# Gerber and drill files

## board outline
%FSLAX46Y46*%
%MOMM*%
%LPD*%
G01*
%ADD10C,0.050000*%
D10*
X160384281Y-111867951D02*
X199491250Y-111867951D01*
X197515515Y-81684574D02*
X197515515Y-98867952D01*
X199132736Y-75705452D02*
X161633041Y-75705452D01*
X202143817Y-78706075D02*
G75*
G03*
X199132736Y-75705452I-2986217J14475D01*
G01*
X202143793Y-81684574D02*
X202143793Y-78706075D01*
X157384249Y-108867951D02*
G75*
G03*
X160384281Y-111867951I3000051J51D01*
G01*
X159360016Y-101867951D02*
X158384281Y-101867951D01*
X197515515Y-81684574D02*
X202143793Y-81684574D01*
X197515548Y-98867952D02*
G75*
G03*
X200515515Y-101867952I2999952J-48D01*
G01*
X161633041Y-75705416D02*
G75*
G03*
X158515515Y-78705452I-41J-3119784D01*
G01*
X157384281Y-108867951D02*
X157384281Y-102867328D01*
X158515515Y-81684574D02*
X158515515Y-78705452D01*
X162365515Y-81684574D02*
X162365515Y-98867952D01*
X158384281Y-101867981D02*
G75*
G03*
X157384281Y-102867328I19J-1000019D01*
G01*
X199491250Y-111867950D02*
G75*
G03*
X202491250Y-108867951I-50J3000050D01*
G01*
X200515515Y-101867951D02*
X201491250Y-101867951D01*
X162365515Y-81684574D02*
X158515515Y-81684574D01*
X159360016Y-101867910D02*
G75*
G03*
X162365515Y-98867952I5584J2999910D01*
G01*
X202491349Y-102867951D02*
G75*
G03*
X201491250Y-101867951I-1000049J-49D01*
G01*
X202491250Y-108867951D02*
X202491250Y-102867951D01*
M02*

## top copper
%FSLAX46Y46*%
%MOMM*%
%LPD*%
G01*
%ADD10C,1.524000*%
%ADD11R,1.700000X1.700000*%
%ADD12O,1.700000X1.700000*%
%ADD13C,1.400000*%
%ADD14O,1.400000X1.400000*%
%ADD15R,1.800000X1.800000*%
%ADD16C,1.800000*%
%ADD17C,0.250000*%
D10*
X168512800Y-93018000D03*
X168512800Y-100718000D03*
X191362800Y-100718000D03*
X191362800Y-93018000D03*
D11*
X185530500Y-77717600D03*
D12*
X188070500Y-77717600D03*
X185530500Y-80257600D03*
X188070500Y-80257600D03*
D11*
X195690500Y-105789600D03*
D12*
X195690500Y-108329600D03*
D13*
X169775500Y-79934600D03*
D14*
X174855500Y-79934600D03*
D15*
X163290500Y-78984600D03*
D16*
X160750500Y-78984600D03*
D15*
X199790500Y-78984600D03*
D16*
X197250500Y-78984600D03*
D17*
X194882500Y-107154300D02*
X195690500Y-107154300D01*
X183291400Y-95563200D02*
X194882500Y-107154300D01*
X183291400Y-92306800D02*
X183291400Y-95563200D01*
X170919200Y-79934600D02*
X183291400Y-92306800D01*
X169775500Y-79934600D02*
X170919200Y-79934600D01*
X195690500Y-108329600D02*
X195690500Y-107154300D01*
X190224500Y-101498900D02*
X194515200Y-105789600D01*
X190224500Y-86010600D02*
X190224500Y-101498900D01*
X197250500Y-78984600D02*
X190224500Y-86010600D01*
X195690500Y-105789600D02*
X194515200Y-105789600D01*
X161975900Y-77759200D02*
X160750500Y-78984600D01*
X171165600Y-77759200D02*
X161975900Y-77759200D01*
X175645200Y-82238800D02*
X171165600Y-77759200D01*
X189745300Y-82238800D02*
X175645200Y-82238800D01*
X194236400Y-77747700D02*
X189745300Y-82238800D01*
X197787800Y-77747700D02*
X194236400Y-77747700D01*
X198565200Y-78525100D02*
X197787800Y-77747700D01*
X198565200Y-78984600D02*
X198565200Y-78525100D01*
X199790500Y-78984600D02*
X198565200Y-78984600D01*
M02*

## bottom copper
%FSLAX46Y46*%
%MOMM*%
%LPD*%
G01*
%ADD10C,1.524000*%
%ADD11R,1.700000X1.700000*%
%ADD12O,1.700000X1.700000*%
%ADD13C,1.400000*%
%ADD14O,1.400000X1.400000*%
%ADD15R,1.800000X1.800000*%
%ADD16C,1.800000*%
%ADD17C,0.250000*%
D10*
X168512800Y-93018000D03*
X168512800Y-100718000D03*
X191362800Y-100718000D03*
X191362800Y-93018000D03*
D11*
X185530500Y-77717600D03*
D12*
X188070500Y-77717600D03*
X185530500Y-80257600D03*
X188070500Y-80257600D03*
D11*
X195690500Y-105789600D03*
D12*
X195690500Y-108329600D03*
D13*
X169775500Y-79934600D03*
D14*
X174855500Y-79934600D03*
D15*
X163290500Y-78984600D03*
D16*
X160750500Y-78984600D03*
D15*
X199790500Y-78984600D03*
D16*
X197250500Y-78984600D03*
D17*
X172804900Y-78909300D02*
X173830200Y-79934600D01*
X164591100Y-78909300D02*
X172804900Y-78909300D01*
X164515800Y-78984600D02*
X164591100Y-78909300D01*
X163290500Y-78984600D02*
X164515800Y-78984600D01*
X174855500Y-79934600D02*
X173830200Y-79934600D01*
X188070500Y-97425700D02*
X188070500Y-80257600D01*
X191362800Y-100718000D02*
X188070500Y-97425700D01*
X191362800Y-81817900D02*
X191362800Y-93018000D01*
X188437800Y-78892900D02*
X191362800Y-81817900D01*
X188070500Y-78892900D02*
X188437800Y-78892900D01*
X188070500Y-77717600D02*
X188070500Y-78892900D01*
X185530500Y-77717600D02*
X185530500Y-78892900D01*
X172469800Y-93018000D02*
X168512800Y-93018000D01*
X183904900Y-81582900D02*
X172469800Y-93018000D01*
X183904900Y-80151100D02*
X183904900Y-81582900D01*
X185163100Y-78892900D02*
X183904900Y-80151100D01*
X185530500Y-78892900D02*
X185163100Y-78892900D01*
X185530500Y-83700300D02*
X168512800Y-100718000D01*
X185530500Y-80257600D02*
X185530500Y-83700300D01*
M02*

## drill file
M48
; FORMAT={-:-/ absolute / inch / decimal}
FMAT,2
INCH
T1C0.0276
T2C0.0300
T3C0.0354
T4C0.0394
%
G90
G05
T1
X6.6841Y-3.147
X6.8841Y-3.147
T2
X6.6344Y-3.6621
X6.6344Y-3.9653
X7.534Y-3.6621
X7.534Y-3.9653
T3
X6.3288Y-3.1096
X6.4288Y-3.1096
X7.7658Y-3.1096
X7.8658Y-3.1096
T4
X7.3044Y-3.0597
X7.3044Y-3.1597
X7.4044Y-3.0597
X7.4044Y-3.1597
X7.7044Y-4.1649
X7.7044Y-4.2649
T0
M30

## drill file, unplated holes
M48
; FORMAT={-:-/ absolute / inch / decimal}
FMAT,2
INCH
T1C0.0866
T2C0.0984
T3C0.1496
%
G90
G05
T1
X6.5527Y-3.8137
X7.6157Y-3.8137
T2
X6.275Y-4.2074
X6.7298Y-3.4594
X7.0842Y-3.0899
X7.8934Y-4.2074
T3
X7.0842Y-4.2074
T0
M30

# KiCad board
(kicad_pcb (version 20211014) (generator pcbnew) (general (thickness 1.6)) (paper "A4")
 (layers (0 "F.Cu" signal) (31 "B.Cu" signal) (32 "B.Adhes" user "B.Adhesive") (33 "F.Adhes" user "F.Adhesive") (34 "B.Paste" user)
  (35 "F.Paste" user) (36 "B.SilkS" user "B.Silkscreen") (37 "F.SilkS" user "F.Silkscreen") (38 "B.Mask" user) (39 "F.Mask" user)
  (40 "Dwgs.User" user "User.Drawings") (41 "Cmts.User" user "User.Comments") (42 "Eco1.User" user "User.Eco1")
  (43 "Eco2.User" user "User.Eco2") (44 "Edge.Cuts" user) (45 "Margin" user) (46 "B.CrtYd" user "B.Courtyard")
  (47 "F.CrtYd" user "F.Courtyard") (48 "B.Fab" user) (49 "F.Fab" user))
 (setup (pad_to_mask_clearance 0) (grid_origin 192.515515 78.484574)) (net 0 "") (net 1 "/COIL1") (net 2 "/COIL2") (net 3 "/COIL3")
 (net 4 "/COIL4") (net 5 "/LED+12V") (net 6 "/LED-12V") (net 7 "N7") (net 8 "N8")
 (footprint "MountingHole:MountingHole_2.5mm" (layer "F.Cu") (at 179.9378 78.4846)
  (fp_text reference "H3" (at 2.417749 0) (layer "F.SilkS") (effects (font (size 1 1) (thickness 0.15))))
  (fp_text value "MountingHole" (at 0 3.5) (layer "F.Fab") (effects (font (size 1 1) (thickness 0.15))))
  (pad "" np_thru_hole circle locked (at 0 0) (size 2.5 2.5) (drill 2.5) (layers *.Cu *.Mask)))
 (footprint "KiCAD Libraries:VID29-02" (layer "F.Cu") (at 180.1028 96.868)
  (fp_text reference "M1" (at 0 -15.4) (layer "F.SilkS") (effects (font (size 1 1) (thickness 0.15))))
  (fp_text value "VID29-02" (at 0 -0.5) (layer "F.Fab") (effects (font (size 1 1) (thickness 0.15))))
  (pad "" np_thru_hole circle locked (at -9.165 -9) (size 2.5 2.5) (drill 2.5) (layers *.Cu *.Mask))
  (pad "" np_thru_hole circle locked (at 13.335 0) (size 2.2 2.2) (drill 2.2) (layers *.Cu *.Mask))
  (pad "" np_thru_hole circle locked (at -0.165 10) (size 3.8 3.8) (drill 3.8) (layers *.Cu *.Mask))
  (pad "" np_thru_hole circle locked (at -13.665 0) (size 2.2 2.2) (drill 2.2) (layers *.Cu *.Mask))
  (pad "1" thru_hole circle locked (at -11.59 -3.85) (size 1.524 1.524) (drill 0.762) (layers *.Cu *.Mask) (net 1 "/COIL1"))
  (pad "2" thru_hole circle locked (at -11.59 3.85) (size 1.524 1.524) (drill 0.762) (layers *.Cu *.Mask) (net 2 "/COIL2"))
  (pad "3" thru_hole circle locked (at 11.26 3.85) (size 1.524 1.524) (drill 0.762) (layers *.Cu *.Mask) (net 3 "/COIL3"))
  (pad "4" thru_hole circle locked (at 11.26 -3.85) (size 1.524 1.524) (drill 0.762) (layers *.Cu *.Mask) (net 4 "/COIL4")))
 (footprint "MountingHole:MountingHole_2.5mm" (layer "F.Cu") (at 159.3843 106.868)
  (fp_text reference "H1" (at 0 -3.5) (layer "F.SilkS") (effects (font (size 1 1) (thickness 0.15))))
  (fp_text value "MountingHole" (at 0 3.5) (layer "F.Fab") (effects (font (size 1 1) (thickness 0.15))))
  (pad "" np_thru_hole circle locked (at 0 0) (size 2.5 2.5) (drill 2.5) (layers *.Cu *.Mask)))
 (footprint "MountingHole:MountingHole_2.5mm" (layer "F.Cu") (at 200.4913 106.868)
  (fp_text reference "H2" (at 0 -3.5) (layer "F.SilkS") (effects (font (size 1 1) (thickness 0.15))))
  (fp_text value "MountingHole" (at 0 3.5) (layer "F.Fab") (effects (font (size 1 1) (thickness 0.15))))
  (pad "" np_thru_hole circle locked (at 0 0) (size 2.5 2.5) (drill 2.5) (layers *.Cu *.Mask)))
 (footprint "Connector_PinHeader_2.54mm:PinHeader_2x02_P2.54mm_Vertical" (layer "F.Cu") (at 185.5305 77.7176)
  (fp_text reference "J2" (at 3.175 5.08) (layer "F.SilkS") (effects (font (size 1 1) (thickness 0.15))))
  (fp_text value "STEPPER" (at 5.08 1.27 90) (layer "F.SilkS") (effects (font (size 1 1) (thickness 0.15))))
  (pad "1" thru_hole rect locked (at 0 0) (size 1.7 1.7) (drill 1) (layers *.Cu *.Mask) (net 1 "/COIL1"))
  (pad "2" thru_hole oval locked (at 2.54 0) (size 1.7 1.7) (drill 1) (layers *.Cu *.Mask) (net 4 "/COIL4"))
  (pad "3" thru_hole oval locked (at 0 2.54) (size 1.7 1.7) (drill 1) (layers *.Cu *.Mask) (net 2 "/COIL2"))
  (pad "4" thru_hole oval locked (at 2.54 2.54) (size 1.7 1.7) (drill 1) (layers *.Cu *.Mask) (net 3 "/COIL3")))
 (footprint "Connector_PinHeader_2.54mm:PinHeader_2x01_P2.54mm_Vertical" (layer "F.Cu") (at 195.6905 105.7896 -90)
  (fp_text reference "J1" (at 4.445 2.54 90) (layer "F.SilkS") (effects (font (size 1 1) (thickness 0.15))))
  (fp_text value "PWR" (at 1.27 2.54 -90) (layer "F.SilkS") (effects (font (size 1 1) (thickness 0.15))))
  (pad "1" thru_hole rect locked (at 0 0 270) (size 1.7 1.7) (drill 1) (layers *.Cu *.Mask) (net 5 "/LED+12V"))
  (pad "2" thru_hole oval locked (at 2.54 0 270) (size 1.7 1.7) (drill 1) (layers *.Cu *.Mask) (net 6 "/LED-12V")))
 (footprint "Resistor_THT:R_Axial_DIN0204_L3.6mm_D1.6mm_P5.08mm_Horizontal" (layer "F.Cu") (at 169.7755 79.9346)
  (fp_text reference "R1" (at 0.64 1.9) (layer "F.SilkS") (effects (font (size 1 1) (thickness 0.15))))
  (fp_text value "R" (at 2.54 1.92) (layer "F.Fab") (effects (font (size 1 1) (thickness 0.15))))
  (pad "1" thru_hole circle (at 0 0) (size 1.4 1.4) (drill 0.7) (layers *.Cu *.Mask) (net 6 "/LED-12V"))
  (pad "2" thru_hole oval (at 5.08 0) (size 1.4 1.4) (drill 0.7) (layers *.Cu *.Mask) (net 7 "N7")))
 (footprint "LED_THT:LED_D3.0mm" (layer "B.Cu") (at 163.2905 78.9846 180)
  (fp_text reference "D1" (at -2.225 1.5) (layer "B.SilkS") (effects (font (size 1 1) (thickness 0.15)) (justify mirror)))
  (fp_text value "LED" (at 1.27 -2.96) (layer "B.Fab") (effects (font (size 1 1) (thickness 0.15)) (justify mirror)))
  (pad "1" thru_hole rect (at 0 0 180) (size 1.8 1.8) (drill 0.9) (layers *.Cu *.Mask) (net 7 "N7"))
  (pad "2" thru_hole circle (at 2.54 0 180) (size 1.8 1.8) (drill 0.9) (layers *.Cu *.Mask) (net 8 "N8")))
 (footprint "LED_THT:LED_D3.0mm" (layer "B.Cu") (at 199.7905 78.9846 180)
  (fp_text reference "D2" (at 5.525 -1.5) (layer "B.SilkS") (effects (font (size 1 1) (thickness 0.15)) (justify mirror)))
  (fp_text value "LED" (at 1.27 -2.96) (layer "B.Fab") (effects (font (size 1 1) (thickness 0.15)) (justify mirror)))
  (pad "1" thru_hole rect (at 0 0 180) (size 1.8 1.8) (drill 0.9) (layers *.Cu *.Mask) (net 8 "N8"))
  (pad "2" thru_hole circle (at 2.54 0 180) (size 1.8 1.8) (drill 0.9) (layers *.Cu *.Mask) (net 5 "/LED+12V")))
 (gr_line (start 160.384281 111.867951) (end 199.49125 111.867951) (layer "Edge.Cuts") (width 0.05))
 (gr_line (start 197.515515 81.684574) (end 197.515515 98.867952) (layer "Edge.Cuts") (width 0.05))
 (gr_line (start 199.132736 75.705452) (end 161.633041 75.705452) (layer "Edge.Cuts") (width 0.05))
 (gr_arc (start 199.132736 75.705452) (mid 201.265508 76.576339) (end 202.143793 78.706075) (layer "Edge.Cuts") (width 0.05))
 (gr_line (start 202.143793 81.684574) (end 202.143793 78.706075) (layer "Edge.Cuts") (width 0.05))
 (gr_arc (start 160.384281 111.867951) (mid 158.262961 110.989271) (end 157.384281 108.867951) (layer "Edge.Cuts") (width 0.05))
 (gr_line (start 159.360016 101.867951) (end 158.384281 101.867951) (layer "Edge.Cuts") (width 0.05))
 (gr_line (start 197.515515 81.684574) (end 202.143793 81.684574) (layer "Edge.Cuts") (width 0.05))
 (gr_arc (start 200.515515 101.867952) (mid 198.394195 100.989272) (end 197.515515 98.867952) (layer "Edge.Cuts") (width 0.05))
 (gr_arc (start 158.515515 78.705452) (mid 159.469751 76.577243) (end 161.633041 75.705452) (layer "Edge.Cuts") (width 0.05))
 (gr_line (start 157.384281 108.867951) (end 157.384281 102.867328) (layer "Edge.Cuts") (width 0.05))
 (gr_line (start 158.515515 81.684574) (end 158.515515 78.705452) (layer "Edge.Cuts") (width 0.05))
 (gr_line (start 162.365515 81.684574) (end 162.365515 98.867952) (layer "Edge.Cuts") (width 0.05))
 (gr_arc (start 157.384281 102.867328) (mid 157.677399 102.160628) (end 158.384281 101.867951) (layer "Edge.Cuts") (width 0.05))
 (gr_arc (start 202.49125 108.867951) (mid 201.61257 110.989271) (end 199.49125 111.867951) (layer "Edge.Cuts") (width 0.05))
 (gr_line (start 200.515515 101.867951) (end 201.49125 101.867951) (layer "Edge.Cuts") (width 0.05))
 (gr_line (start 162.365515 81.684574) (end 158.515515 81.684574) (layer "Edge.Cuts") (width 0.05))
 (gr_arc (start 162.365515 98.867952) (mid 161.484904 100.991231) (end 159.360016 101.867951) (layer "Edge.Cuts") (width 0.05))
 (gr_arc (start 201.49125 101.867951) (mid 202.198357 102.160844) (end 202.49125 102.867951) (layer "Edge.Cuts") (width 0.05))
 (gr_line (start 202.49125 108.867951) (end 202.49125 102.867951) (layer "Edge.Cuts") (width 0.05))
 (segment (start 185.5305 83.7003) (end 168.5128 100.718) (width 0.25) (layer "B.Cu") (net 2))
 (segment (start 185.5305 80.2576) (end 185.5305 83.7003) (width 0.25) (layer "B.Cu") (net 2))
 (segment (start 185.5305 77.7176) (end 185.5305 78.8929) (width 0.25) (layer "B.Cu") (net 1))
 (segment (start 172.4698 93.018) (end 168.5128 93.018) (width 0.25) (layer "B.Cu") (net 1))
 (segment (start 183.9049 80.1511) (end 183.9049 81.5829) (width 0.25) (layer "B.Cu") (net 1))
 (segment (start 185.1631 78.8929) (end 183.9049 80.1511) (width 0.25) (layer "B.Cu") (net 1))
 (segment (start 185.5305 78.8929) (end 185.1631 78.8929) (width 0.25) (layer "B.Cu") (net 1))
 (segment (start 183.9049 81.5829) (end 172.4698 93.018) (width 0.25) (layer "B.Cu") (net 1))
 (segment (start 191.3628 81.8179) (end 191.3628 93.018) (width 0.25) (layer "B.Cu") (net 4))
 (segment (start 188.4378 78.8929) (end 191.3628 81.8179) (width 0.25) (layer "B.Cu") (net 4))
 (segment (start 188.0705 77.7176) (end 188.0705 78.8929) (width 0.25) (layer "B.Cu") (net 4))
 (segment (start 188.0705 78.8929) (end 188.4378 78.8929) (width 0.25) (layer "B.Cu") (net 4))
 (segment (start 188.0705 97.4257) (end 188.0705 80.2576) (width 0.25) (layer "B.Cu") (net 3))
 (segment (start 191.3628 100.718) (end 188.0705 97.4257) (width 0.25) (layer "B.Cu") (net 3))
 (segment (start 198.5652 78.5251) (end 197.7878 77.7477) (width 0.25) (layer "F.Cu") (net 8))
 (segment (start 197.7878 77.7477) (end 194.2364 77.7477) (width 0.25) (layer "F.Cu") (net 8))
 (segment (start 198.5652 78.9846) (end 198.5652 78.5251) (width 0.25) (layer "F.Cu") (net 8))
 (segment (start 199.7905 78.9846) (end 198.5652 78.9846) (width 0.25) (layer "F.Cu") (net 8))
 (segment (start 194.2364 77.7477) (end 189.7453 82.2388) (width 0.25) (layer "F.Cu") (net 8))
 (segment (start 161.9759 77.7592) (end 160.7505 78.9846) (width 0.25) (layer "F.Cu") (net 8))
 (segment (start 189.7453 82.2388) (end 175.6452 82.2388) (width 0.25) (layer "F.Cu") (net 8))
 (segment (start 171.1656 77.7592) (end 161.9759 77.7592) (width 0.25) (layer "F.Cu") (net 8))
 (segment (start 175.6452 82.2388) (end 171.1656 77.7592) (width 0.25) (layer "F.Cu") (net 8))
 (segment (start 197.2505 78.9846) (end 190.2245 86.0106) (width 0.25) (layer "F.Cu") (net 5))
 (segment (start 195.6905 105.7896) (end 194.5152 105.7896) (width 0.25) (layer "F.Cu") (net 5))
 (segment (start 190.2245 86.0106) (end 190.2245 101.4989) (width 0.25) (layer "F.Cu") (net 5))
 (segment (start 190.2245 101.4989) (end 194.5152 105.7896) (width 0.25) (layer "F.Cu") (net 5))
 (segment (start 170.9192 79.9346) (end 183.2914 92.3068) (width 0.25) (layer "F.Cu") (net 6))
 (segment (start 195.6905 108.3296) (end 195.6905 107.1543) (width 0.25) (layer "F.Cu") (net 6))
 (segment (start 169.7755 79.9346) (end 170.9192 79.9346) (width 0.25) (layer "F.Cu") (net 6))
 (segment (start 183.2914 95.5632) (end 194.8825 107.1543) (width 0.25) (layer "F.Cu") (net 6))
 (segment (start 194.8825 107.1543) (end 195.6905 107.1543) (width 0.25) (layer "F.Cu") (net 6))
 (segment (start 183.2914 92.3068) (end 183.2914 95.5632) (width 0.25) (layer "F.Cu") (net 6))
 (segment (start 174.8555 79.9346) (end 173.8302 79.9346) (width 0.25) (layer "B.Cu") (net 7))
 (segment (start 164.5911 78.9093) (end 172.8049 78.9093) (width 0.25) (layer "B.Cu") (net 7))
 (segment (start 172.8049 78.9093) (end 173.8302 79.9346) (width 0.25) (layer "B.Cu") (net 7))
 (segment (start 163.2905 78.9846) (end 164.5158 78.9846) (width 0.25) (layer "B.Cu") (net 7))
 (segment (start 164.5158 78.9846) (end 164.5911 78.9093) (width 0.25) (layer "B.Cu") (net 7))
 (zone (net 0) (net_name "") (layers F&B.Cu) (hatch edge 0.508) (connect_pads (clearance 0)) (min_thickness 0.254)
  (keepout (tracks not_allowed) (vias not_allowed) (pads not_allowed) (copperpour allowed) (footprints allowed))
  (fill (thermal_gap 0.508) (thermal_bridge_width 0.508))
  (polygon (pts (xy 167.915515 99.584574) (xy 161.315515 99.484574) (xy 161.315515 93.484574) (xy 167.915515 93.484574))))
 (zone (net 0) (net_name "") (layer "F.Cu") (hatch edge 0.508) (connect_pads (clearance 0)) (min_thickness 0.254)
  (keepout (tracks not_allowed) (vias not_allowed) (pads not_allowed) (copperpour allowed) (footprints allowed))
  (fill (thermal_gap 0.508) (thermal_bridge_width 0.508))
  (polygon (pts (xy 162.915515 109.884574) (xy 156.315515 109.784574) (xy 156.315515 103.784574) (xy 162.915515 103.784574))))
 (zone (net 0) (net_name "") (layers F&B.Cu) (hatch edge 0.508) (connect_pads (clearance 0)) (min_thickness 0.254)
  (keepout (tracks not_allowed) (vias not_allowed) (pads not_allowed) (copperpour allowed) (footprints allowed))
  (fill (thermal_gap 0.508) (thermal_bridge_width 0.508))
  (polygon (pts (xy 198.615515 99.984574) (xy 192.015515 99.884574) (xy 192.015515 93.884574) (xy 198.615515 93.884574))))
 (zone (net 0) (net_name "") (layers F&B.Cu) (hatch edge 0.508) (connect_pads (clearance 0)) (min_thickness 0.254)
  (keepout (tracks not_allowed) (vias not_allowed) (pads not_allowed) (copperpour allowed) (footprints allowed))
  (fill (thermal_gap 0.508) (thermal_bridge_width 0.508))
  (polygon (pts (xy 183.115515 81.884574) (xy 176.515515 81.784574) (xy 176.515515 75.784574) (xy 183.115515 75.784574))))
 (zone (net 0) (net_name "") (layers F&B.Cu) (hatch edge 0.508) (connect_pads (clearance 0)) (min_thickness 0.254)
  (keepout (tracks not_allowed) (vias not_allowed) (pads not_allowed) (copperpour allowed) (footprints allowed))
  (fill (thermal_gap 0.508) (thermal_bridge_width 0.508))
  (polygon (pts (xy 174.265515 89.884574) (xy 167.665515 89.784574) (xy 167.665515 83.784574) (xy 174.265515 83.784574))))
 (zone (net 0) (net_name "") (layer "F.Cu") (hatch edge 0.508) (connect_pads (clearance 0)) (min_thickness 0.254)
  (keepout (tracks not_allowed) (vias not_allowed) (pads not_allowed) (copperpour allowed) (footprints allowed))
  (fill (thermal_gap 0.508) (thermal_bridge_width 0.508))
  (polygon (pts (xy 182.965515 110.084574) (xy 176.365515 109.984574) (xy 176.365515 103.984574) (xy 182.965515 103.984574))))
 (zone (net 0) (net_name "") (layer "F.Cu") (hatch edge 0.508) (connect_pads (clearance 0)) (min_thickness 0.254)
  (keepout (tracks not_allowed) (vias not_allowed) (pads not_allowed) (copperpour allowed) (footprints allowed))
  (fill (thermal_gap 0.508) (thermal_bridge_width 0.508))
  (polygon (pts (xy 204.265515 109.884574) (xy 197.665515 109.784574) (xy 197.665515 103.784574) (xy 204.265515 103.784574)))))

